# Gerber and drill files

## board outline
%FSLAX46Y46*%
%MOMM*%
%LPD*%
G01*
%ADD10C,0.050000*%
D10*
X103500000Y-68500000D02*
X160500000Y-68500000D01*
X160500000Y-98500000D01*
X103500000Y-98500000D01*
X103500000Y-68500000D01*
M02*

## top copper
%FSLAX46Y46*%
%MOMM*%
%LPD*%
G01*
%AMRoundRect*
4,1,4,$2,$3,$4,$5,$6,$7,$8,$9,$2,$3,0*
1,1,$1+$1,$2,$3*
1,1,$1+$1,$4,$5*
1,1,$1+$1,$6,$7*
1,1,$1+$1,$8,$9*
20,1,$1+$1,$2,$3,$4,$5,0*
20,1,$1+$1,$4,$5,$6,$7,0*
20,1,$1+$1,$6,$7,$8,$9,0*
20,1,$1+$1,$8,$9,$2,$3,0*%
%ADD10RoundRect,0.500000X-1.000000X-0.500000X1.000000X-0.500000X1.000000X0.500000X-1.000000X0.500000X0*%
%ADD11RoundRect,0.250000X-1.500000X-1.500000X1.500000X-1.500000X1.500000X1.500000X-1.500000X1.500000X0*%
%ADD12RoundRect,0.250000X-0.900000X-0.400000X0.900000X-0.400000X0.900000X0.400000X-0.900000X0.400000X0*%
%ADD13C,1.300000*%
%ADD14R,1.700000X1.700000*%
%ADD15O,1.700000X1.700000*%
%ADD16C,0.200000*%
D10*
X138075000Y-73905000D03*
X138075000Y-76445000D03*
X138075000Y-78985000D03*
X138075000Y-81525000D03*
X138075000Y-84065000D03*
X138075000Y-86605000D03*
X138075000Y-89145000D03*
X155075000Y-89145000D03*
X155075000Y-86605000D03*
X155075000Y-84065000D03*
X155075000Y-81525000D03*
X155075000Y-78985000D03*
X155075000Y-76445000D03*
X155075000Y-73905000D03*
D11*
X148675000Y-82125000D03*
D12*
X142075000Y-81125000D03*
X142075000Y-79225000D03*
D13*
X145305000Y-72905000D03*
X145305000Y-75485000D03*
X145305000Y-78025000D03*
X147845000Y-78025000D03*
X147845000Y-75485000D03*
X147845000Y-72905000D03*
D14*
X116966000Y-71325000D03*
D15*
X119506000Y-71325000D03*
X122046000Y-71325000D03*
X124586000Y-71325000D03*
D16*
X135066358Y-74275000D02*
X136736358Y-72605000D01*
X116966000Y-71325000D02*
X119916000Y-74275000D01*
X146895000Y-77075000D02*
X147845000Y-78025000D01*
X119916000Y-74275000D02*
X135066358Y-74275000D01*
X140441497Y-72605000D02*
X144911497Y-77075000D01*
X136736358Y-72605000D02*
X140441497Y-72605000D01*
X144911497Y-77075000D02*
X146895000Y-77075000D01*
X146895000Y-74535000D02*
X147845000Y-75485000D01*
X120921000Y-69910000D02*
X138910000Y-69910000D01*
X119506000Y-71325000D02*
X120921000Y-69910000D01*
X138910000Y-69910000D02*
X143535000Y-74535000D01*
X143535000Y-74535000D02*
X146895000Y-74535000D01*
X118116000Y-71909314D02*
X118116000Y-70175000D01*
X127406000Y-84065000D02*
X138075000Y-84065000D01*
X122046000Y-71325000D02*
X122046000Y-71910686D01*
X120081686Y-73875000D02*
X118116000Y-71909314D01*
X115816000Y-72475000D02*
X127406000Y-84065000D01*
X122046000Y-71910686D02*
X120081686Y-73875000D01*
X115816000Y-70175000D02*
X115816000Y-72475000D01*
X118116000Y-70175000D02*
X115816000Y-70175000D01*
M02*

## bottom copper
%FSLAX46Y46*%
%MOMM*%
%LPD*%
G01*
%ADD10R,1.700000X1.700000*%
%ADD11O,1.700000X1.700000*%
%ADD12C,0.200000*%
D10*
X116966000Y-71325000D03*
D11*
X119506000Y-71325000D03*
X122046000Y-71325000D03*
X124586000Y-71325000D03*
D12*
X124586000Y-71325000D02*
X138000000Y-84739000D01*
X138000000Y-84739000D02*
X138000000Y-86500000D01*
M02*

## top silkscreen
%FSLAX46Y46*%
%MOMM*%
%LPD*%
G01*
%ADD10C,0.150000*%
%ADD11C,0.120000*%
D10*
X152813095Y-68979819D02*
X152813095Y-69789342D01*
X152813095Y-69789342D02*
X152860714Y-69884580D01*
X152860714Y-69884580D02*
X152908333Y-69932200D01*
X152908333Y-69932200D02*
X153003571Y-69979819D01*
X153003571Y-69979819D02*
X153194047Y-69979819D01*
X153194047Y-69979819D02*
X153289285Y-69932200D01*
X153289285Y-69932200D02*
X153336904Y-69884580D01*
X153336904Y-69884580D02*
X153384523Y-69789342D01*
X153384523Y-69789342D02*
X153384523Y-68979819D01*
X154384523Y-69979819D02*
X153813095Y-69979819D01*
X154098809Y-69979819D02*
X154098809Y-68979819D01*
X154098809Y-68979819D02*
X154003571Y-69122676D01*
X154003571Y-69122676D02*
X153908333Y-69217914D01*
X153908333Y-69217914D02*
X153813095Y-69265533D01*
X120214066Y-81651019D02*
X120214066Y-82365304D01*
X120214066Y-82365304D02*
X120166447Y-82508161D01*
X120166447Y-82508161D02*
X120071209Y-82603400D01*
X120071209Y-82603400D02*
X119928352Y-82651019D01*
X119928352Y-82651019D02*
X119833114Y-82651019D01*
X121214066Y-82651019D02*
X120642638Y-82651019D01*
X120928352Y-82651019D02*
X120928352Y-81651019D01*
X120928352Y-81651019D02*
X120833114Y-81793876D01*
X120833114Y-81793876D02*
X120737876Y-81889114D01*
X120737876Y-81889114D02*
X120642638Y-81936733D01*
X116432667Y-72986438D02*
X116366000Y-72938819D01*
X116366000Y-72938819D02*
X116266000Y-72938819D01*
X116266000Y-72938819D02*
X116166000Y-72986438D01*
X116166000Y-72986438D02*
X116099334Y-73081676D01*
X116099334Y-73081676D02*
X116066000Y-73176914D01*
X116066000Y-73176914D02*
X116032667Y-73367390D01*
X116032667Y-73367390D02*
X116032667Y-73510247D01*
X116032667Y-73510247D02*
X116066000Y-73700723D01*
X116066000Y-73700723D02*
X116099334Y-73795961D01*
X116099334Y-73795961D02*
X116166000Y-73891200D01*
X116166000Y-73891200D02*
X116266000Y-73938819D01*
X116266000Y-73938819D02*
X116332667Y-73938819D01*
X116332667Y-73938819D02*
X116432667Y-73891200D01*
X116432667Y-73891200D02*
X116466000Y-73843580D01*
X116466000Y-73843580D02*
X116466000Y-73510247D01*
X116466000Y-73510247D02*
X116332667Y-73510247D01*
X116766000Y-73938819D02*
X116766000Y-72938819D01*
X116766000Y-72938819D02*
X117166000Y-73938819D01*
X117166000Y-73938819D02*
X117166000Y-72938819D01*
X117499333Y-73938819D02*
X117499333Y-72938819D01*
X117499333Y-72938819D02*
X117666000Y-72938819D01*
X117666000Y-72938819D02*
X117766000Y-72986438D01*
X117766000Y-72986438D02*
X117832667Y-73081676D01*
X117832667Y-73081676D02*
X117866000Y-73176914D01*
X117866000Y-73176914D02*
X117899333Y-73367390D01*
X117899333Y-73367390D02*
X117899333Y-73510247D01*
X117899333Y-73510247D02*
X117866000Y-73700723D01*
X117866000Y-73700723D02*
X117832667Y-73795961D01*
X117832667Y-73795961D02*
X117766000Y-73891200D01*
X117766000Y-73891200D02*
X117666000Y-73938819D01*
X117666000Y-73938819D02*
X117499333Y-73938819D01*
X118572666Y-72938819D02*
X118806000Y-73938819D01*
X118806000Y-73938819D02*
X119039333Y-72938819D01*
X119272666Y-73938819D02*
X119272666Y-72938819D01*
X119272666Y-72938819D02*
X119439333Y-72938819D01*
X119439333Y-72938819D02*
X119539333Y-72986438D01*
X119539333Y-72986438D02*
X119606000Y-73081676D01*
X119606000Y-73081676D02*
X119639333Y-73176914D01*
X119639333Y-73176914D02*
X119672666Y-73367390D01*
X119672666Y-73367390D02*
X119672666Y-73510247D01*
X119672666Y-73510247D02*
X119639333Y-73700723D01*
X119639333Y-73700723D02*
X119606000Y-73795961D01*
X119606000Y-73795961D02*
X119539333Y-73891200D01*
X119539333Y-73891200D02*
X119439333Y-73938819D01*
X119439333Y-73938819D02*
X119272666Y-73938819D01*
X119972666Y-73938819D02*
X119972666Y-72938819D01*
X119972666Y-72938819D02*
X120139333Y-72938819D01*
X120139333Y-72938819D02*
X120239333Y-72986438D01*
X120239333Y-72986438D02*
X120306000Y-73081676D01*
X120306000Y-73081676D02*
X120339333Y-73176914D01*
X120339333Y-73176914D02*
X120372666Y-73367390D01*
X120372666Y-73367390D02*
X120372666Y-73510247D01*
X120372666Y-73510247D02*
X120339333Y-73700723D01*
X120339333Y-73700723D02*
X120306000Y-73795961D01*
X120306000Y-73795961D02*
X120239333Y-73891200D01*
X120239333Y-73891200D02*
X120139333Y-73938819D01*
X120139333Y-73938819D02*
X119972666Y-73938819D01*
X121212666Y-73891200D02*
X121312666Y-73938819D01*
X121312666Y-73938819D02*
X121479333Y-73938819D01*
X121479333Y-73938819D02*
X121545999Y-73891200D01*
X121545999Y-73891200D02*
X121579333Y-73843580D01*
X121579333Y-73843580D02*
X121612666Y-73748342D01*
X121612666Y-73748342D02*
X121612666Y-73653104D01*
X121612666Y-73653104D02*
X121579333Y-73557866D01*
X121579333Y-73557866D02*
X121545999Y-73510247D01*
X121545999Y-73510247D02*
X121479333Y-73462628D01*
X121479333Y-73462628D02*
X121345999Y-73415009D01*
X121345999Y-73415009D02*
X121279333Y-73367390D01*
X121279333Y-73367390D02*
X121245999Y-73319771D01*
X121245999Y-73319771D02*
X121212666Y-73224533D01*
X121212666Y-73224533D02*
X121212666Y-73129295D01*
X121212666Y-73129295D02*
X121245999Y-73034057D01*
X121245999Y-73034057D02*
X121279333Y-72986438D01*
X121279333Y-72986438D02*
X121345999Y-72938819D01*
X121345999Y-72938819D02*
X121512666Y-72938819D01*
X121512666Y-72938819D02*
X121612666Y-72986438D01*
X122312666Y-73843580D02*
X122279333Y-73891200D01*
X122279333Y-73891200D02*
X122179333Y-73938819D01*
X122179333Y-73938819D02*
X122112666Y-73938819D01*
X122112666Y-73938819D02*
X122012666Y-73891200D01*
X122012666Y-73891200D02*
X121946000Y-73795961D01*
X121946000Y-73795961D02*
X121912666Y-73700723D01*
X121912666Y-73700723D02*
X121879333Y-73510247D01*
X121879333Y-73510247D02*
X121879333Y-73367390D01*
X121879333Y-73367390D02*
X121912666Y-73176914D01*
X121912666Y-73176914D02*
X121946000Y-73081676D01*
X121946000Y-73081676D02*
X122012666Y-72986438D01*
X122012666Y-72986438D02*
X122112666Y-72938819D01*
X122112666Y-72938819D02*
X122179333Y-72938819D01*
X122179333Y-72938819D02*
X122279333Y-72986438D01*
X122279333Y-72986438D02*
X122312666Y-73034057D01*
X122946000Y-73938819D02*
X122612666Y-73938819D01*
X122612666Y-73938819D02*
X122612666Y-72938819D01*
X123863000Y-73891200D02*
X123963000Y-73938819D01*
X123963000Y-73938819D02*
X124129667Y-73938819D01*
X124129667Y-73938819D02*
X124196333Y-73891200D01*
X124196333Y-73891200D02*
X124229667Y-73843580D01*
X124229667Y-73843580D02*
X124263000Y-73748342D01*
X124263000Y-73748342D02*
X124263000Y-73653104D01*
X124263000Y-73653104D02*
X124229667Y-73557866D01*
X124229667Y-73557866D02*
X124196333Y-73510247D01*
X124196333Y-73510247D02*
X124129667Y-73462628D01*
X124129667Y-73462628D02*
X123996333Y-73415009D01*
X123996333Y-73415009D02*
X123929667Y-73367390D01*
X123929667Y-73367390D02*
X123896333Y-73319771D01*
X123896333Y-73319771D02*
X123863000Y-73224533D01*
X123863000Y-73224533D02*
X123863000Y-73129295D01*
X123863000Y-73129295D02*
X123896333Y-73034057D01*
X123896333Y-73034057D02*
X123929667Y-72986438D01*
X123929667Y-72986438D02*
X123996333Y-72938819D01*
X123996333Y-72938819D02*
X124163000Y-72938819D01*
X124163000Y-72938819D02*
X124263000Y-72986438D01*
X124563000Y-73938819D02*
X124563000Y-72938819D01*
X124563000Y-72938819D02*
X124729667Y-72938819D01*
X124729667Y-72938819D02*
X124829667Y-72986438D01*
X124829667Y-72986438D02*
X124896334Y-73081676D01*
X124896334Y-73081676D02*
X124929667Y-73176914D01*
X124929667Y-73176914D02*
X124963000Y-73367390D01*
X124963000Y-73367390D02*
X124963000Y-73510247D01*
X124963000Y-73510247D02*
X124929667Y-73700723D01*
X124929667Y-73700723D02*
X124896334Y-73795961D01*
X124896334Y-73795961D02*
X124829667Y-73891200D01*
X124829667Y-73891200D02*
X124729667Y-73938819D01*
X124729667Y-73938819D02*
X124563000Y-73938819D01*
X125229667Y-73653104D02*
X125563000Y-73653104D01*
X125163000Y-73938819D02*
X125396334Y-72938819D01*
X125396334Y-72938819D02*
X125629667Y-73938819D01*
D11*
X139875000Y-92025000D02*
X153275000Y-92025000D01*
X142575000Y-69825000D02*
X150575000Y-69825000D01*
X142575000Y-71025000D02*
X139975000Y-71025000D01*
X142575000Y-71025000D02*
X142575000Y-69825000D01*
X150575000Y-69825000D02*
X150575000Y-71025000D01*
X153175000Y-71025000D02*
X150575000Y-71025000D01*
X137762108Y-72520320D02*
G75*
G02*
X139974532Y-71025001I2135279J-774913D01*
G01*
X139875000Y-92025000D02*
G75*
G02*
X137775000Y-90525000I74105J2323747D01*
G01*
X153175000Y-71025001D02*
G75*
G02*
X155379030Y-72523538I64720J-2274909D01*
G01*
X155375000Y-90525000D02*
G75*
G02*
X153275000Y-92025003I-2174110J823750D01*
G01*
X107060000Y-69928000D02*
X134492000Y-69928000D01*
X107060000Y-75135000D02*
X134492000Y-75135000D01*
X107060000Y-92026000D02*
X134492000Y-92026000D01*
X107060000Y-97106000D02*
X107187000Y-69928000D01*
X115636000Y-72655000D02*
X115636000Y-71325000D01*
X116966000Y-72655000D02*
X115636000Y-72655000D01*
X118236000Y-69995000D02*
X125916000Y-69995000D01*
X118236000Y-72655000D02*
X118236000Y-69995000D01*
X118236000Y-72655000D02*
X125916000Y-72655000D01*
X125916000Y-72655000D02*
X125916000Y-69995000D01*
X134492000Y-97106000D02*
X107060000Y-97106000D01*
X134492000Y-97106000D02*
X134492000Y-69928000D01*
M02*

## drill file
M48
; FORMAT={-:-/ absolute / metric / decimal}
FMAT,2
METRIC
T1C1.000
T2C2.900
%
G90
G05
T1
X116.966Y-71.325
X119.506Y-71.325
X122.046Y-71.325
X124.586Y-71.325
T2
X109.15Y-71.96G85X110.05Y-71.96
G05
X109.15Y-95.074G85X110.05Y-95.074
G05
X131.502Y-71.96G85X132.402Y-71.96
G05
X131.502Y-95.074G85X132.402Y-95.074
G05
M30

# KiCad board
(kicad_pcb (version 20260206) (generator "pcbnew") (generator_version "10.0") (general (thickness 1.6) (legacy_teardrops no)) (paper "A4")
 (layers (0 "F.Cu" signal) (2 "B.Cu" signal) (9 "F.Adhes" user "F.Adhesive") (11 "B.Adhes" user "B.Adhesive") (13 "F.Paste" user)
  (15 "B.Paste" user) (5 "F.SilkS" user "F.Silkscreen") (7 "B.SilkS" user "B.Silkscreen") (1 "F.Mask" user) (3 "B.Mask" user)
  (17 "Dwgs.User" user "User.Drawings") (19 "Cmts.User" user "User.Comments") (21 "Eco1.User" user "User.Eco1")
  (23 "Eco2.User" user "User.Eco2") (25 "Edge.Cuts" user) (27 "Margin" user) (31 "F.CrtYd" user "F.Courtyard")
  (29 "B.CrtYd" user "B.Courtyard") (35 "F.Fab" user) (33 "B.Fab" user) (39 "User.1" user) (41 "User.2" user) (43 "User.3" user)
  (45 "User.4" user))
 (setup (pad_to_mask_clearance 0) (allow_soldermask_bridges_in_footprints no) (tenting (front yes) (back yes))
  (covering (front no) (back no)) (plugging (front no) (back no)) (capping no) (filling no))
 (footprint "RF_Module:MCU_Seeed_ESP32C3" (layer "F.Cu") (at 146.575 81.525)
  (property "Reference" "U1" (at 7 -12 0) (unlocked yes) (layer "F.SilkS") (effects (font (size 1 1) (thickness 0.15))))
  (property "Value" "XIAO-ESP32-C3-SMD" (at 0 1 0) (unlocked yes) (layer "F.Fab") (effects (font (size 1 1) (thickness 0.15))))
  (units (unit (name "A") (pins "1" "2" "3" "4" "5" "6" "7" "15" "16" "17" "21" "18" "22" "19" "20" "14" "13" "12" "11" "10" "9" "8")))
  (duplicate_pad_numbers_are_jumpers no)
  (fp_line (start -6.7 10.5) (end 6.7 10.5) (stroke (width 0.12) (type default)) (layer "F.SilkS"))
  (fp_line (start -4 -11.7) (end 4 -11.7) (stroke (width 0.12) (type default)) (layer "F.SilkS"))
  (fp_line (start -4 -10.5) (end -6.6 -10.5) (stroke (width 0.12) (type default)) (layer "F.SilkS"))
  (fp_line (start -4 -10.5) (end -4 -11.7) (stroke (width 0.12) (type default)) (layer "F.SilkS"))
  (fp_line (start 4 -11.7) (end 4 -10.5) (stroke (width 0.12) (type default)) (layer "F.SilkS"))
  (fp_line (start 6.6 -10.5) (end 4 -10.5) (stroke (width 0.12) (type default)) (layer "F.SilkS"))
  (fp_arc (start -8.812892 -9.00468) (mid -7.949609 -10.111769) (end -6.600468 -10.499999) (stroke (width 0.12) (type default))
   (layer "F.SilkS"))
  (fp_arc (start -6.7 10.5) (mid -7.977232 10.068125) (end -8.8 9) (stroke (width 0.12) (type default)) (layer "F.SilkS"))
  (fp_arc (start 6.6 -10.499999) (mid 7.944325 -10.107116) (end 8.804034 -9.001464) (stroke (width 0.12) (type default)) (layer "F.SilkS"))
  (fp_arc (start 8.8 9) (mid 7.977232 10.068125) (end 6.7 10.5) (stroke (width 0.12) (type default)) (layer "F.SilkS"))
  (pad "" smd roundrect (at 1.1 -0.4) (size 1.5 1.5) (layers "F.Paste") (roundrect_rratio 0.1666666667))
  (pad "" smd roundrect (at 1.1 1.6) (size 1.5 1.5) (layers "F.Paste") (roundrect_rratio 0.1666666667))
  (pad "" smd roundrect (at 3.1 -0.4) (size 1.5 1.5) (layers "F.Paste") (roundrect_rratio 0.1666666667))
  (pad "" smd roundrect (at 3.1 1.6) (size 1.5 1.5) (layers "F.Paste") (roundrect_rratio 0.1666666667))
  (pad "1" smd roundrect (at -8.5 -7.62) (size 3 2) (layers "F.Cu" "F.Mask" "F.Paste") (roundrect_rratio 0.25)
   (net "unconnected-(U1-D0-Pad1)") (thermal_bridge_angle 45))
  (pad "2" smd roundrect (at -8.5 -5.08) (size 3 2) (layers "F.Cu" "F.Mask" "F.Paste") (roundrect_rratio 0.25)
   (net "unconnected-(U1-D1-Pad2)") (thermal_bridge_angle 45))
  (pad "3" smd roundrect (at -8.5 -2.54) (size 3 2) (layers "F.Cu" "F.Mask" "F.Paste") (roundrect_rratio 0.25)
   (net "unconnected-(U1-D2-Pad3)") (thermal_bridge_angle 45))
  (pad "4" smd roundrect (at -8.5 0) (size 3 2) (layers "F.Cu" "F.Mask" "F.Paste") (roundrect_rratio 0.25) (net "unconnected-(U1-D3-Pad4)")
   (thermal_bridge_angle 45))
  (pad "5" smd roundrect (at -8.5 2.54) (size 3 2) (layers "F.Cu" "F.Mask" "F.Paste") (roundrect_rratio 0.25) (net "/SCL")
   (thermal_bridge_angle 45))
  (pad "6" smd roundrect (at -8.5 5.08) (size 3 2) (layers "F.Cu" "F.Mask" "F.Paste") (roundrect_rratio 0.25) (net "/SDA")
   (thermal_bridge_angle 45))
  (pad "7" smd roundrect (at -8.5 7.62) (size 3 2) (layers "F.Cu" "F.Mask" "F.Paste") (roundrect_rratio 0.25)
   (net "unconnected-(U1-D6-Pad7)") (thermal_bridge_angle 45))
  (pad "8" smd roundrect (at 8.5 7.62) (size 3 2) (layers "F.Cu" "F.Mask" "F.Paste") (roundrect_rratio 0.25)
   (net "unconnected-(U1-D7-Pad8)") (thermal_bridge_angle 45))
  (pad "9" smd roundrect (at 8.5 5.08) (size 3 2) (layers "F.Cu" "F.Mask" "F.Paste") (roundrect_rratio 0.25)
   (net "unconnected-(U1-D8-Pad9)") (thermal_bridge_angle 45))
  (pad "10" smd roundrect (at 8.5 2.54) (size 3 2) (layers "F.Cu" "F.Mask" "F.Paste") (roundrect_rratio 0.25)
   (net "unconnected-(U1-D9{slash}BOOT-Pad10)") (thermal_bridge_angle 45))
  (pad "11" smd roundrect (at 8.5 0) (size 3 2) (layers "F.Cu" "F.Mask" "F.Paste") (roundrect_rratio 0.25)
   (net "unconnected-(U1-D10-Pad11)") (thermal_bridge_angle 45))
  (pad "12" smd roundrect (at 8.5 -2.54) (size 3 2) (layers "F.Cu" "F.Mask" "F.Paste") (roundrect_rratio 0.25)
   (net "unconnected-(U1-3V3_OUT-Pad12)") (thermal_bridge_angle 45))
  (pad "13" smd roundrect (at 8.5 -5.08) (size 3 2) (layers "F.Cu" "F.Mask" "F.Paste") (roundrect_rratio 0.25)
   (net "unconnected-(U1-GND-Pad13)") (thermal_bridge_angle 45))
  (pad "14" smd roundrect (at 8.5 -7.62) (size 3 2) (layers "F.Cu" "F.Mask" "F.Paste") (roundrect_rratio 0.25)
   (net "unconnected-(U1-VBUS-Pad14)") (thermal_bridge_angle 45))
  (pad "15" smd roundrect (at 2.1 0.6) (size 3.5 3.5) (layers "F.Cu" "F.Mask") (roundrect_rratio 0.07142857143)
   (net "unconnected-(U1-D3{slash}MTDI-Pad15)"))
  (pad "16" smd roundrect (at -4.5 -0.4) (size 2.3 1.3) (layers "F.Cu" "F.Mask" "F.Paste") (roundrect_rratio 0.1923076923)
   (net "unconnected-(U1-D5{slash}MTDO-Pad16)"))
  (pad "17" smd roundrect (at -4.5 -2.3) (size 2.3 1.3) (layers "F.Cu" "F.Mask" "F.Paste") (roundrect_rratio 0.1923076923)
   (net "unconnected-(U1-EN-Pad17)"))
  (pad "18" smd circle (at -1.27 -8.62) (size 1.3 1.3) (layers "F.Cu" "F.Mask" "F.Paste") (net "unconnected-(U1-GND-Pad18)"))
  (pad "19" smd circle (at -1.27 -6.04) (size 1.3 1.3) (layers "F.Cu" "F.Mask" "F.Paste") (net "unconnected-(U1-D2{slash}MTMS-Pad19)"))
  (pad "20" smd circle (at -1.27 -3.5) (size 1.3 1.3) (layers "F.Cu" "F.Mask" "F.Paste") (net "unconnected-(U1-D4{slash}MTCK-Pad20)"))
  (pad "21" smd circle (at 1.27 -3.5) (size 1.3 1.3) (layers "F.Cu" "F.Mask" "F.Paste") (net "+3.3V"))
  (pad "22" smd circle (at 1.27 -6.04) (size 1.3 1.3) (layers "F.Cu" "F.Mask" "F.Paste") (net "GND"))
  (pad "23" smd circle (at 1.27 -8.62) (size 1.3 1.3) (layers "F.Cu" "F.Mask" "F.Paste")))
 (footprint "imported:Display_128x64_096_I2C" (layer "F.Cu") (at 120.776 71.325)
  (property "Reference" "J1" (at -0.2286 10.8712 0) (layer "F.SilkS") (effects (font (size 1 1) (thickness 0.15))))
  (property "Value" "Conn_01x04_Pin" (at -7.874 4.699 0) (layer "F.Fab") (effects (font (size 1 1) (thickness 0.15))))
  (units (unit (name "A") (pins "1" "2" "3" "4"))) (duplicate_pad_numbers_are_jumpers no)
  (fp_line (start -13.716 -1.397) (end 13.716 -1.397) (stroke (width 0.12) (type solid)) (layer "F.SilkS"))
  (fp_line (start -13.716 3.81) (end 13.716 3.81) (stroke (width 0.12) (type solid)) (layer "F.SilkS"))
  (fp_line (start -13.716 20.701) (end 13.716 20.701) (stroke (width 0.12) (type solid)) (layer "F.SilkS"))
  (fp_line (start -13.716 25.781) (end -13.589 -1.397) (stroke (width 0.12) (type solid)) (layer "F.SilkS"))
  (fp_line (start -5.14 1.33) (end -5.14 0) (stroke (width 0.12) (type solid)) (layer "F.SilkS"))
  (fp_line (start -3.81 1.33) (end -5.14 1.33) (stroke (width 0.12) (type solid)) (layer "F.SilkS"))
  (fp_line (start -2.54 -1.33) (end 5.14 -1.33) (stroke (width 0.12) (type solid)) (layer "F.SilkS"))
  (fp_line (start -2.54 1.33) (end -2.54 -1.33) (stroke (width 0.12) (type solid)) (layer "F.SilkS"))
  (fp_line (start -2.54 1.33) (end 5.14 1.33) (stroke (width 0.12) (type solid)) (layer "F.SilkS"))
  (fp_line (start 5.14 1.33) (end 5.14 -1.33) (stroke (width 0.12) (type solid)) (layer "F.SilkS"))
  (fp_line (start 13.716 25.781) (end -13.716 25.781) (stroke (width 0.12) (type solid)) (layer "F.SilkS"))
  (fp_line (start 13.716 25.781) (end 13.716 -1.397) (stroke (width 0.12) (type solid)) (layer "F.SilkS"))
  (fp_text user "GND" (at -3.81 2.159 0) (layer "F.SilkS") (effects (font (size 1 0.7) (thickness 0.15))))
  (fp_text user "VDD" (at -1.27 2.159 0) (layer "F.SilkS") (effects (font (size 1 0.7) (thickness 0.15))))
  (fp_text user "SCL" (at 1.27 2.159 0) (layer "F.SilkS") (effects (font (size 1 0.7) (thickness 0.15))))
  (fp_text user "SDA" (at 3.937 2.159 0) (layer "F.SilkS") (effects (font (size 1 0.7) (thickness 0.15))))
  (pad "" np_thru_hole oval (at -11.176 0.635) (size 3.8 2.9) (drill oval 3.8 2.9) (layers "*.Cu" "*.Mask"))
  (pad "" np_thru_hole oval (at -11.176 23.749) (size 3.8 2.9) (drill oval 3.8 2.9) (layers "*.Cu" "*.Mask"))
  (pad "" np_thru_hole oval (at 11.176 0.635) (size 3.8 2.9) (drill oval 3.8 2.9) (layers "*.Cu" "*.Mask"))
  (pad "" np_thru_hole oval (at 11.176 23.749) (size 3.8 2.9) (drill oval 3.8 2.9) (layers "*.Cu" "*.Mask"))
  (pad "1" thru_hole rect (at -3.81 0 90) (size 1.7 1.7) (drill 1) (layers "*.Cu" "*.Mask") (remove_unused_layers no) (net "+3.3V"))
  (pad "2" thru_hole oval (at -1.27 0 90) (size 1.7 1.7) (drill 1) (layers "*.Cu" "*.Mask") (remove_unused_layers no) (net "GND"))
  (pad "3" thru_hole oval (at 1.27 0 90) (size 1.7 1.7) (drill 1) (layers "*.Cu" "*.Mask") (remove_unused_layers no) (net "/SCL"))
  (pad "4" thru_hole oval (at 3.81 0 90) (size 1.7 1.7) (drill 1) (layers "*.Cu" "*.Mask") (remove_unused_layers no) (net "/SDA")))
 (gr_rect (start 103.5 68.5) (end 160.5 98.5) (stroke (width 0.05) (type default)) (fill no) (layer "Edge.Cuts"))
 (segment (start 135.066358 74.275) (end 136.736358 72.605) (width 0.2) (layer "F.Cu") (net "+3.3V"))
 (segment (start 116.966 71.325) (end 119.916 74.275) (width 0.2) (layer "F.Cu") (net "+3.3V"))
 (segment (start 146.895 77.075) (end 147.845 78.025) (width 0.2) (layer "F.Cu") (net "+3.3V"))
 (segment (start 119.916 74.275) (end 135.066358 74.275) (width 0.2) (layer "F.Cu") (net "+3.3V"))
 (segment (start 140.441497 72.605) (end 144.911497 77.075) (width 0.2) (layer "F.Cu") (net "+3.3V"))
 (segment (start 136.736358 72.605) (end 140.441497 72.605) (width 0.2) (layer "F.Cu") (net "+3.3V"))
 (segment (start 144.911497 77.075) (end 146.895 77.075) (width 0.2) (layer "F.Cu") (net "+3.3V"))
 (segment (start 146.895 74.535) (end 147.845 75.485) (width 0.2) (layer "F.Cu") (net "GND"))
 (segment (start 120.921 69.91) (end 138.91 69.91) (width 0.2) (layer "F.Cu") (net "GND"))
 (segment (start 119.506 71.325) (end 120.921 69.91) (width 0.2) (layer "F.Cu") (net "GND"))
 (segment (start 138.91 69.91) (end 143.535 74.535) (width 0.2) (layer "F.Cu") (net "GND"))
 (segment (start 143.535 74.535) (end 146.895 74.535) (width 0.2) (layer "F.Cu") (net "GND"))
 (segment (start 124.586 71.325) (end 138 84.739) (width 0.2) (layer "B.Cu") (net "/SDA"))
 (segment (start 138 84.739) (end 138 86.5) (width 0.2) (layer "B.Cu") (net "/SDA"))
 (segment (start 118.116 71.909314) (end 118.116 70.175) (width 0.2) (layer "F.Cu") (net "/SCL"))
 (segment (start 127.406 84.065) (end 138.075 84.065) (width 0.2) (layer "F.Cu") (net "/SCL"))
 (segment (start 122.046 71.325) (end 122.046 71.910686) (width 0.2) (layer "F.Cu") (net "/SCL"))
 (segment (start 120.081686 73.875) (end 118.116 71.909314) (width 0.2) (layer "F.Cu") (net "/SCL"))
 (segment (start 115.816 72.475) (end 127.406 84.065) (width 0.2) (layer "F.Cu") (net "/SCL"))
 (segment (start 122.046 71.910686) (end 120.081686 73.875) (width 0.2) (layer "F.Cu") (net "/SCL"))
 (segment (start 115.816 70.175) (end 115.816 72.475) (width 0.2) (layer "F.Cu") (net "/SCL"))
 (segment (start 118.116 70.175) (end 115.816 70.175) (width 0.2) (layer "F.Cu") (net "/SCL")))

